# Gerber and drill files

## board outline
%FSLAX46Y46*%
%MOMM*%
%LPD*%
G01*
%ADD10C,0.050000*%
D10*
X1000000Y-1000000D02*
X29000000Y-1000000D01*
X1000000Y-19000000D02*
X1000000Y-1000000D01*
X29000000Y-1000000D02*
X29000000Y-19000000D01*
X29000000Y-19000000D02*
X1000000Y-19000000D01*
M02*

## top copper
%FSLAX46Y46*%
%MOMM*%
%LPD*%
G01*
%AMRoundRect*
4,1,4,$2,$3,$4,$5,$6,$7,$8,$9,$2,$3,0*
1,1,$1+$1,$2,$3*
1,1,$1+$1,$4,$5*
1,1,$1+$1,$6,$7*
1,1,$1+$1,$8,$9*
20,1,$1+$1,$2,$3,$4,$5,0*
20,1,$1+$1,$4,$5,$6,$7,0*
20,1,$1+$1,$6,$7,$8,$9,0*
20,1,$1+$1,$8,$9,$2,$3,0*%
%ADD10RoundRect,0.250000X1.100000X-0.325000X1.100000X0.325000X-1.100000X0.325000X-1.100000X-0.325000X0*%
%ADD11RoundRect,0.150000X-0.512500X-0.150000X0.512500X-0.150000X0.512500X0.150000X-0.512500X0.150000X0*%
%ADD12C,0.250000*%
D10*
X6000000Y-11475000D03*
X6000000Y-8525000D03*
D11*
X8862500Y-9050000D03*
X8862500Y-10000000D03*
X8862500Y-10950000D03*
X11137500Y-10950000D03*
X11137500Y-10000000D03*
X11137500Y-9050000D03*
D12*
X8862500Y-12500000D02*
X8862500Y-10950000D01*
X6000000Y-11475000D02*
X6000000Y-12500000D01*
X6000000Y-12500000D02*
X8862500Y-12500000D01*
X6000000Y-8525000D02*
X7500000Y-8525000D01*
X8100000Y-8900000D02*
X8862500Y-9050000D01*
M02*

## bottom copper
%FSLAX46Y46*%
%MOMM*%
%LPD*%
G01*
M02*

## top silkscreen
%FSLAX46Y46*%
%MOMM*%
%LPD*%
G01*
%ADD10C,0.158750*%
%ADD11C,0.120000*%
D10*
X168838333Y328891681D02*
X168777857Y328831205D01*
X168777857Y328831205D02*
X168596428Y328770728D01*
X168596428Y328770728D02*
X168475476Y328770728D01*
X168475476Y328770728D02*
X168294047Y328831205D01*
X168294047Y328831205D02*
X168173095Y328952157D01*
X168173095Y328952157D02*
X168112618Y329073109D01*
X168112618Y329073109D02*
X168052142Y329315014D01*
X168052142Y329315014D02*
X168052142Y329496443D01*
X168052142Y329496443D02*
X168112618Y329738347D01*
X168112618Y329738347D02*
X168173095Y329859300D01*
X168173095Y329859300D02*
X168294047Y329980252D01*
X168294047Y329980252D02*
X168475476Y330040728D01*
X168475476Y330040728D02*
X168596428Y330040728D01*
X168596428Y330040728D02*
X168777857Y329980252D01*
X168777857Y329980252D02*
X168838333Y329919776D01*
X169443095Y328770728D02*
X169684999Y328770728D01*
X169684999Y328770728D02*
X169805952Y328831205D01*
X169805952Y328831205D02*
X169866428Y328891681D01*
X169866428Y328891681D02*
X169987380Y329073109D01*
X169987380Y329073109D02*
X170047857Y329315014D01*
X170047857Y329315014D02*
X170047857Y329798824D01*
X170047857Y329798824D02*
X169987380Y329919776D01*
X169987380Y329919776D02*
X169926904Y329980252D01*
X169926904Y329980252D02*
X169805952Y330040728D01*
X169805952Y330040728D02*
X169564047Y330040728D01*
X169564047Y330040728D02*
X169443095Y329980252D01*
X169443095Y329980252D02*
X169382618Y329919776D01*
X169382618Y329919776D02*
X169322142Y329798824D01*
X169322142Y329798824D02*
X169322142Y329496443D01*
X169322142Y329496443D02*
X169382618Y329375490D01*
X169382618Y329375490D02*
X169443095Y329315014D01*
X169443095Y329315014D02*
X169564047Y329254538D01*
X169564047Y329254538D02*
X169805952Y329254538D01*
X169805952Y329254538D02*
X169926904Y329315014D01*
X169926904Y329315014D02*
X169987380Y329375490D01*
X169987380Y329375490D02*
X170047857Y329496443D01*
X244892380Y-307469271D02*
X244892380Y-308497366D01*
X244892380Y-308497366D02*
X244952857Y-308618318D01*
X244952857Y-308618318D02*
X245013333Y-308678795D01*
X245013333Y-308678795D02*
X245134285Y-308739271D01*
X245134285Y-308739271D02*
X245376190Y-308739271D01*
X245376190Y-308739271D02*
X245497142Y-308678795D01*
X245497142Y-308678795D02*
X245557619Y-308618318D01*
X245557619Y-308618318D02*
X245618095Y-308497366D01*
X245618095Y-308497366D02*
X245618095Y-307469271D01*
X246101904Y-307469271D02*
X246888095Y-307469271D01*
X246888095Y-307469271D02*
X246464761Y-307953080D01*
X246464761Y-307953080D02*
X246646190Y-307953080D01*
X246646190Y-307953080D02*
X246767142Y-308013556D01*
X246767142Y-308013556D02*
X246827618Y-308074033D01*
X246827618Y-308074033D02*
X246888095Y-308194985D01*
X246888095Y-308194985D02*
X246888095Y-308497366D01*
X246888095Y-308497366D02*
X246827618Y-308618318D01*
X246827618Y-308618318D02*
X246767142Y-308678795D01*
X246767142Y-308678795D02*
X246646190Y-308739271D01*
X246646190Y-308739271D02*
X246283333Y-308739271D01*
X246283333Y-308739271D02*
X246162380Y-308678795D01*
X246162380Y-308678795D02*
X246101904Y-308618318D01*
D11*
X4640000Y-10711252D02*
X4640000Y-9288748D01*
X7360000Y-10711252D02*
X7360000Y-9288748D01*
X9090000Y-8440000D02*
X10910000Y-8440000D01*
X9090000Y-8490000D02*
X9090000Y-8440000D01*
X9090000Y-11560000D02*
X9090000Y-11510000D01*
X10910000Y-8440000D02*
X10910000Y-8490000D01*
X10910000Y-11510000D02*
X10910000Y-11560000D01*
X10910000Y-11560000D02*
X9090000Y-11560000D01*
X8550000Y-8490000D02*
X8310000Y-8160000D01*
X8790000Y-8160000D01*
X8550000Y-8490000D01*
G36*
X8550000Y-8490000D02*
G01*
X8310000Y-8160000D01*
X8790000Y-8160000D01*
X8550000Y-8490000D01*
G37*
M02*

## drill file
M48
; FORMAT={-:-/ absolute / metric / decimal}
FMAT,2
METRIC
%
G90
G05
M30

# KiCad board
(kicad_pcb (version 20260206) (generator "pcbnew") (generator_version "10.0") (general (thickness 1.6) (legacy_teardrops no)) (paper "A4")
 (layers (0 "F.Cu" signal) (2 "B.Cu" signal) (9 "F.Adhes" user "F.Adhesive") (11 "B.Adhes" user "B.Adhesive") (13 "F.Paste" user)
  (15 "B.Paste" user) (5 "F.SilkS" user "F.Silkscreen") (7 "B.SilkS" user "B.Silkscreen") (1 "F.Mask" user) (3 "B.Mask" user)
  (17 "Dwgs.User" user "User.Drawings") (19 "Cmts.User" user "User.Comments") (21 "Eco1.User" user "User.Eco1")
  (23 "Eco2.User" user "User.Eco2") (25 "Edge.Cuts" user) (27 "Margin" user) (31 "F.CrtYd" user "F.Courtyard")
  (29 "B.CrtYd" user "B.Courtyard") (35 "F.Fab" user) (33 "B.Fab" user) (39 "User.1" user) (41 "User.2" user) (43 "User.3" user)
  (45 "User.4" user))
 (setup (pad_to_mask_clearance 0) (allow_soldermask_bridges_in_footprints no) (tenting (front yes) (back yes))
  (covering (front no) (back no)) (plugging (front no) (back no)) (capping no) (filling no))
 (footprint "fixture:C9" (layer "F.Cu") (at 6 10 90)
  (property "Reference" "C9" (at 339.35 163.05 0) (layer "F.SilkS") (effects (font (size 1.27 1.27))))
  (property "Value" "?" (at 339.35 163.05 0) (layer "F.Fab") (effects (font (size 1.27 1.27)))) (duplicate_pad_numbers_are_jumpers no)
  (fp_line (start -0.711252 -1.36) (end 0.711252 -1.36) (stroke (width 0.12) (type solid)) (layer "F.SilkS"))
  (fp_line (start -0.711252 1.36) (end 0.711252 1.36) (stroke (width 0.12) (type solid)) (layer "F.SilkS"))
  (pad "1" smd roundrect (at -1.475 0 90) (size 1.15 2.7) (layers "F.Cu" "F.Mask" "F.Paste") (roundrect_rratio 0.217391) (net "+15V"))
  (pad "2" smd roundrect (at 1.475 0 90) (size 1.15 2.7) (layers "F.Cu" "F.Mask" "F.Paste") (roundrect_rratio 0.217391) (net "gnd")))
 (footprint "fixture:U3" (layer "F.Cu") (at 10 10)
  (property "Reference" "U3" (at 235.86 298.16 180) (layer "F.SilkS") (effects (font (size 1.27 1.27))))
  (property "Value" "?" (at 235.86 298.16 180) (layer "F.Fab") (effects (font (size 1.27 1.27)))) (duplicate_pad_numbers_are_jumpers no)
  (fp_line (start -0.91 -1.56) (end 0.91 -1.56) (stroke (width 0.12) (type solid)) (layer "F.SilkS"))
  (fp_line (start -0.91 -1.51) (end -0.91 -1.56) (stroke (width 0.12) (type solid)) (layer "F.SilkS"))
  (fp_line (start -0.91 1.56) (end -0.91 1.51) (stroke (width 0.12) (type solid)) (layer "F.SilkS"))
  (fp_line (start 0.91 -1.56) (end 0.91 -1.51) (stroke (width 0.12) (type solid)) (layer "F.SilkS"))
  (fp_line (start 0.91 1.51) (end 0.91 1.56) (stroke (width 0.12) (type solid)) (layer "F.SilkS"))
  (fp_line (start 0.91 1.56) (end -0.91 1.56) (stroke (width 0.12) (type solid)) (layer "F.SilkS"))
  (fp_poly (pts (xy -1.45 -1.51) (xy -1.69 -1.84) (xy -1.21 -1.84)) (stroke (width 0.12) (type solid)) (fill yes) (layer "F.SilkS"))
  (pad "1" smd roundrect (at -1.1375 -0.95) (size 1.325 0.6) (layers "F.Cu" "F.Mask" "F.Paste") (roundrect_rratio 0.25) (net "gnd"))
  (pad "2" smd roundrect (at -1.1375 0) (size 1.325 0.6) (layers "F.Cu" "F.Mask" "F.Paste") (roundrect_rratio 0.25) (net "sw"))
  (pad "3" smd roundrect (at -1.1375 0.95) (size 1.325 0.6) (layers "F.Cu" "F.Mask" "F.Paste") (roundrect_rratio 0.25) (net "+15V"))
  (pad "4" smd roundrect (at 1.1375 0.95) (size 1.325 0.6) (layers "F.Cu" "F.Mask" "F.Paste") (roundrect_rratio 0.25) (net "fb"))
  (pad "5" smd roundrect (at 1.1375 0) (size 1.325 0.6) (layers "F.Cu" "F.Mask" "F.Paste") (roundrect_rratio 0.25) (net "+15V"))
  (pad "6" smd roundrect (at 1.1375 -0.95) (size 1.325 0.6) (layers "F.Cu" "F.Mask" "F.Paste") (roundrect_rratio 0.25) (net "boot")))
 (gr_line (start 1 1) (end 29 1) (stroke (width 0.05) (type default)) (layer "Edge.Cuts"))
 (gr_line (start 1 19) (end 1 1) (stroke (width 0.05) (type default)) (layer "Edge.Cuts"))
 (gr_line (start 29 1) (end 29 19) (stroke (width 0.05) (type default)) (layer "Edge.Cuts"))
 (gr_line (start 29 19) (end 1 19) (stroke (width 0.05) (type default)) (layer "Edge.Cuts"))
 (segment (start 8.8625 12.5) (end 8.8625 10.95) (width 0.25) (layer "F.Cu") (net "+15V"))
 (segment (start 6 11.475) (end 6 12.5) (width 0.25) (layer "F.Cu") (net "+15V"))
 (segment (start 6 12.5) (end 8.8625 12.5) (width 0.25) (layer "F.Cu") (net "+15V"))
 (segment (start 6 8.525) (end 7.5 8.525) (width 0.25) (layer "F.Cu") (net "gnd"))
 (segment (start 8.1 8.9) (end 8.8625 9.05) (width 0.25) (layer "F.Cu") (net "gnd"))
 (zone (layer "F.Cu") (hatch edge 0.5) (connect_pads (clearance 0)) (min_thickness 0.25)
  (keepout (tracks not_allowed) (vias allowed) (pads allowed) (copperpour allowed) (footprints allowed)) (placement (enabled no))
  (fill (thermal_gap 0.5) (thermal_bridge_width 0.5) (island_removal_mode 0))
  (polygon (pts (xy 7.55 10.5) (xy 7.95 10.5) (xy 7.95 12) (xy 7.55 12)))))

